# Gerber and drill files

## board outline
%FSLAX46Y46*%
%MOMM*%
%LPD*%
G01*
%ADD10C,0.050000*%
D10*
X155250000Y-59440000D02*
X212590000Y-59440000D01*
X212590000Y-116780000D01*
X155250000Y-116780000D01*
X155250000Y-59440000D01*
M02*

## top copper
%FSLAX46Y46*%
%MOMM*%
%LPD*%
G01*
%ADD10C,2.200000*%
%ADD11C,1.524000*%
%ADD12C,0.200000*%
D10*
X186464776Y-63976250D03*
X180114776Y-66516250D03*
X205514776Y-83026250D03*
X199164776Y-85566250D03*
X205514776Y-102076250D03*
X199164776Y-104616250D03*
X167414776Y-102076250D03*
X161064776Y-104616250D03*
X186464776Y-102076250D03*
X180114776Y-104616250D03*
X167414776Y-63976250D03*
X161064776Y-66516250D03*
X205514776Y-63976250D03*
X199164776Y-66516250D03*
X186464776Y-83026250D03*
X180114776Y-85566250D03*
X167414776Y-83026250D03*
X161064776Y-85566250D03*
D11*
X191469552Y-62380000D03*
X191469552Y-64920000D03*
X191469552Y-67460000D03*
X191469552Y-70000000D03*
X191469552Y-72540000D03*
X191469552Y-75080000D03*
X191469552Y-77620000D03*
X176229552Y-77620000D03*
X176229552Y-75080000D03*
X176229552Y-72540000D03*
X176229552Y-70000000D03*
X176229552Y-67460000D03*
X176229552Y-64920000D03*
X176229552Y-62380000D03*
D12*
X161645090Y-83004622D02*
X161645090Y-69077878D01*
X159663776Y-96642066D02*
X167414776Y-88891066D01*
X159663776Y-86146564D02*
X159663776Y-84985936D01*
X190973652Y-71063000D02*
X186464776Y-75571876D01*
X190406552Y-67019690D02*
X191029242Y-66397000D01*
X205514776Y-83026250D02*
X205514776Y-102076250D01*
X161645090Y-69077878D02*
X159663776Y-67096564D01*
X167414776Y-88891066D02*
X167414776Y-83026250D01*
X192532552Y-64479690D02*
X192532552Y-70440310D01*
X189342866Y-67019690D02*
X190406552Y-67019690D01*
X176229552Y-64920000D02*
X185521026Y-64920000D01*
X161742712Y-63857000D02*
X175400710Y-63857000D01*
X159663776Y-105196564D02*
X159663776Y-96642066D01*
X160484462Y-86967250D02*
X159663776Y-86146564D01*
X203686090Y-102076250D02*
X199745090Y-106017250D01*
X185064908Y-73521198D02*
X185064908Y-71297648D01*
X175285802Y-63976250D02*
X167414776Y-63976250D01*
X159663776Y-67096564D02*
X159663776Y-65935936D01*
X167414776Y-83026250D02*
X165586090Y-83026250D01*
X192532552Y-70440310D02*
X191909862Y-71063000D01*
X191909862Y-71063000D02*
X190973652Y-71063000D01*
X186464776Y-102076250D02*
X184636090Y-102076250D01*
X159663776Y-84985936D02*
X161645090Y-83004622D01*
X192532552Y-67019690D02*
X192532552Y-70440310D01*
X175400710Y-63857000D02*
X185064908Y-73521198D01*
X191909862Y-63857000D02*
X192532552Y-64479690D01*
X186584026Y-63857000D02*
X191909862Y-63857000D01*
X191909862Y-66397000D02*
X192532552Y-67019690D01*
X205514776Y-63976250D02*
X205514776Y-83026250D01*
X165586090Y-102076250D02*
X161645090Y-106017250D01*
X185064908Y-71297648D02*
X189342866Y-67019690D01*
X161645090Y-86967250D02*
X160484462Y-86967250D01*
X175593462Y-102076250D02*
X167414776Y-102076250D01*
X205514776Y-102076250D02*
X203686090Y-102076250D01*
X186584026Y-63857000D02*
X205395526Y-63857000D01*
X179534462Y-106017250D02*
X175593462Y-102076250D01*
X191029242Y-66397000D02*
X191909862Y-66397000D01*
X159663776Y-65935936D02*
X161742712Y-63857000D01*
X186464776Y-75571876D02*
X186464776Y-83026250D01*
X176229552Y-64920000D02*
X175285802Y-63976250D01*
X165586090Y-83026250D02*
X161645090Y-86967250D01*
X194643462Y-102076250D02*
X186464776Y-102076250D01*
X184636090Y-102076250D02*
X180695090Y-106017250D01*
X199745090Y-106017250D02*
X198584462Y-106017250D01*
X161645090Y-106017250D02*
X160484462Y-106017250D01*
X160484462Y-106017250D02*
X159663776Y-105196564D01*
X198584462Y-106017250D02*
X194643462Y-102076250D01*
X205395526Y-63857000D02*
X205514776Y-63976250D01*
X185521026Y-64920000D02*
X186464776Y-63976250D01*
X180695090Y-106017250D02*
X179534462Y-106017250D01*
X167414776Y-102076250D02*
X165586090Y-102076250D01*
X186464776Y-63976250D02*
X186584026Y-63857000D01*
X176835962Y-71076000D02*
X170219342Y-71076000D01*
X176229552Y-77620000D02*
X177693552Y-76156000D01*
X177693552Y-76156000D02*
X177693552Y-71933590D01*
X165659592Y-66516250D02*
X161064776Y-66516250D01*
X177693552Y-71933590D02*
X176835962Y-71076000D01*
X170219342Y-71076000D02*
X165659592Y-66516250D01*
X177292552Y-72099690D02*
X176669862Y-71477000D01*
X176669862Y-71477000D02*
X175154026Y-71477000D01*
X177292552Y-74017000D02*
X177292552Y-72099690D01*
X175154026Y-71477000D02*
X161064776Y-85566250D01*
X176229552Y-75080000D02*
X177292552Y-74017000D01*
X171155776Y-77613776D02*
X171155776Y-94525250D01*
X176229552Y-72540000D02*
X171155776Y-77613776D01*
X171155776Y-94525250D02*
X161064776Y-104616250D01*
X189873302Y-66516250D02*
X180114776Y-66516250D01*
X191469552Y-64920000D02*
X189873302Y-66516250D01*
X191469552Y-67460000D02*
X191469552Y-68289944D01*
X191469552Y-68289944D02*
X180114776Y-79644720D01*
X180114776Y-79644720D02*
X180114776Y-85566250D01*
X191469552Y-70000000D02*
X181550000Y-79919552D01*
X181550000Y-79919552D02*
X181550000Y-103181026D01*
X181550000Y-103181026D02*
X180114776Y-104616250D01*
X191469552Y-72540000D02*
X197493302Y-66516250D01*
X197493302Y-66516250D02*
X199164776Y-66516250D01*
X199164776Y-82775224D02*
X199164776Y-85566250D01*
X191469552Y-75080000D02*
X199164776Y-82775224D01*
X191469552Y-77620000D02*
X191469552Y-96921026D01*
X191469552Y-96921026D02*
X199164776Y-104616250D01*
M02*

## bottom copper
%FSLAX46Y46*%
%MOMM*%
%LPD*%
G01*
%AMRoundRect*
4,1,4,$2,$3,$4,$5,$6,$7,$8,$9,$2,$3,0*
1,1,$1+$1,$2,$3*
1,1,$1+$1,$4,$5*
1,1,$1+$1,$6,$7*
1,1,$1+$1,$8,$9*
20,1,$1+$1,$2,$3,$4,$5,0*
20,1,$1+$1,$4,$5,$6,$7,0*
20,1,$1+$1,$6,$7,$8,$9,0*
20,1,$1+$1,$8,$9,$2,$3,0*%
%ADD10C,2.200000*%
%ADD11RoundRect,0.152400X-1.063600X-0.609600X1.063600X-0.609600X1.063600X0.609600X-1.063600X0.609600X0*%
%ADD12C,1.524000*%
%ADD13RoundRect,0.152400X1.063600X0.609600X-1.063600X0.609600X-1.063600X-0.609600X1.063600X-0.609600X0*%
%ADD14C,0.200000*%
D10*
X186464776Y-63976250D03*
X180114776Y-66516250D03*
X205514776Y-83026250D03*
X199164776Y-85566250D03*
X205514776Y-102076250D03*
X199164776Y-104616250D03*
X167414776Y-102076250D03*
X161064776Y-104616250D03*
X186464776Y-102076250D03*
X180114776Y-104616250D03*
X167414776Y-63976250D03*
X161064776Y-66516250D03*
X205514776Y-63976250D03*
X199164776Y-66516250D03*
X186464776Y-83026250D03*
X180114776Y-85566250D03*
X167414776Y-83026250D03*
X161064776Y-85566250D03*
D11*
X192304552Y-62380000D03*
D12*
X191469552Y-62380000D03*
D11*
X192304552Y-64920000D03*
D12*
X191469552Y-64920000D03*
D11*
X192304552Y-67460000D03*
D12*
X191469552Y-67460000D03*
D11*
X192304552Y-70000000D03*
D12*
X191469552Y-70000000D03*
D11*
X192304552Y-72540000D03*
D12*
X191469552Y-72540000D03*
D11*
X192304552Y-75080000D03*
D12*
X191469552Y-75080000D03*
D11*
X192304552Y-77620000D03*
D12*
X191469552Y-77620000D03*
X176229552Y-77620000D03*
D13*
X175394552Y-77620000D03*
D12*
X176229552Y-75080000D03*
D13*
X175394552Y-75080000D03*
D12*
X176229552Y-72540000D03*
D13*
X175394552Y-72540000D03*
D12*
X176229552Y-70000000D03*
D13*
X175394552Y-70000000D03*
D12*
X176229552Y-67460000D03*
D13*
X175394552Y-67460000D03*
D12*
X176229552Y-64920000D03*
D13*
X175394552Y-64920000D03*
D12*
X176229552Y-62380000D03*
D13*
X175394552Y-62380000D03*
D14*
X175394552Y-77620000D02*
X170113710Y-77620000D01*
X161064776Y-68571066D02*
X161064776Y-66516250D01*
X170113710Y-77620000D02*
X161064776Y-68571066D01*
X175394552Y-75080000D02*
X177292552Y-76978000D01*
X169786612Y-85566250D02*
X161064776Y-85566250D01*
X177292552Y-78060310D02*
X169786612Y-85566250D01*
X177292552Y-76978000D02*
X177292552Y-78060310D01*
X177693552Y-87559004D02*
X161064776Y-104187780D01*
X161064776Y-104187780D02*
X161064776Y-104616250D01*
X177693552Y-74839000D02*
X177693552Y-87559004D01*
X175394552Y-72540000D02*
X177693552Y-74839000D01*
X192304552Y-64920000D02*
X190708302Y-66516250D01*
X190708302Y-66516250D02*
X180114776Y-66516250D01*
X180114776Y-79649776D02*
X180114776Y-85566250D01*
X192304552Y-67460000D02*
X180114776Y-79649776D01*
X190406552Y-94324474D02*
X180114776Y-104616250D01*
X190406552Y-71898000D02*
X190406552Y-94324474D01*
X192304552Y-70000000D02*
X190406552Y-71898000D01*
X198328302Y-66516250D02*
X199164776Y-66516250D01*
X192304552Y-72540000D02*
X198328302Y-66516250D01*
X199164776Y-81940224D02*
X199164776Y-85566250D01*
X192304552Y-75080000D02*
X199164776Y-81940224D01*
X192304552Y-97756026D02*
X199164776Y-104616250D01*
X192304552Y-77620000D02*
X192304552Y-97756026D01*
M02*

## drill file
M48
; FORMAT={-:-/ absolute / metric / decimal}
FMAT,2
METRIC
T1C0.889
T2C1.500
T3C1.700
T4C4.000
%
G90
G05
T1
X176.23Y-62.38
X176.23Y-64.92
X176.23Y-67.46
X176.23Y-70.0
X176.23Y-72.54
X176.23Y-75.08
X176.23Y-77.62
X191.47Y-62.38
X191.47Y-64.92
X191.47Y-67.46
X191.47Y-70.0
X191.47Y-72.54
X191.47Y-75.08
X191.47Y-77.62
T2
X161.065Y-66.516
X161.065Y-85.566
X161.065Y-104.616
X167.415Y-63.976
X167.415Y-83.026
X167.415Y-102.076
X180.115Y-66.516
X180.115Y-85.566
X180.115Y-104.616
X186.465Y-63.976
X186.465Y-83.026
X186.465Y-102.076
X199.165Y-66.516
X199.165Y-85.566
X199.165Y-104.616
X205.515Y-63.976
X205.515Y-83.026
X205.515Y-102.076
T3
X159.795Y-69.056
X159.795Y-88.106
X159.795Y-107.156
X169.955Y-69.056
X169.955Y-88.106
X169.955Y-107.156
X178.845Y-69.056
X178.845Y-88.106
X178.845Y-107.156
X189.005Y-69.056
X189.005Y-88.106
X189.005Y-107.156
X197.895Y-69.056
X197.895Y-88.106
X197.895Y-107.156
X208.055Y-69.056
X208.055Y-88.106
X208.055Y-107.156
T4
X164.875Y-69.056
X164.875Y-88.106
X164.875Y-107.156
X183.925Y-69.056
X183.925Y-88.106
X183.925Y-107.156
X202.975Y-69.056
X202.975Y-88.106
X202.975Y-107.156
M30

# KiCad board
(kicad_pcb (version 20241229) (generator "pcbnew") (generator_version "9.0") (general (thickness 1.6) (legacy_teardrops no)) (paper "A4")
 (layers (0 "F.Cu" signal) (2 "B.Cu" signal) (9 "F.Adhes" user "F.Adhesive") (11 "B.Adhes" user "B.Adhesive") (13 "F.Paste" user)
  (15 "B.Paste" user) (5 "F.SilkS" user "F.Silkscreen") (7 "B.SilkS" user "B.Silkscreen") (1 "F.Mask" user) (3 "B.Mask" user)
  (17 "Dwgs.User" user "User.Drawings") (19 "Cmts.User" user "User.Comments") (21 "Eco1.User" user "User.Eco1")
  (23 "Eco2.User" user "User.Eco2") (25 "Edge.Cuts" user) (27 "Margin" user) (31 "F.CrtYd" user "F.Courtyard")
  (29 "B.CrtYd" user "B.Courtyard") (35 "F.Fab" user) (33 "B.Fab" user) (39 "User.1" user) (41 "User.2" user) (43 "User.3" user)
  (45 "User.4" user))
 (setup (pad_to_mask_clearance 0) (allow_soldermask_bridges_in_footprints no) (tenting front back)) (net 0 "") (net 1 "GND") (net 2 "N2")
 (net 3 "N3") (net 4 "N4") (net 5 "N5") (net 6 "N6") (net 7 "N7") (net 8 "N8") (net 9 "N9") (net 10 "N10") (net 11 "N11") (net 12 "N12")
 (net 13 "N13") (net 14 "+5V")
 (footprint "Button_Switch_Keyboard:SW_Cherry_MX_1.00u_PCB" (layer "F.Cu") (at 186.464776 63.97625)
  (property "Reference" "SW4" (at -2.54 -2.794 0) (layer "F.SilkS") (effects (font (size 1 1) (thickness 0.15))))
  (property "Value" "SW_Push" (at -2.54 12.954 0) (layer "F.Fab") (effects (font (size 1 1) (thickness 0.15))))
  (pad "" np_thru_hole circle (at -7.62 5.08) (size 1.7 1.7) (drill 1.7) (layers "*.Cu" "*.Mask"))
  (pad "" np_thru_hole circle (at -2.54 5.08) (size 4 4) (drill 4) (layers "*.Cu" "*.Mask"))
  (pad "" np_thru_hole circle (at 2.54 5.08) (size 1.7 1.7) (drill 1.7) (layers "*.Cu" "*.Mask"))
  (pad "1" thru_hole circle (at 0 0) (size 2.2 2.2) (drill 1.5) (layers "*.Cu" "*.Mask") (remove_unused_layers no) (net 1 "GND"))
  (pad "2" thru_hole circle (at -6.35 2.54) (size 2.2 2.2) (drill 1.5) (layers "*.Cu" "*.Mask") (remove_unused_layers no) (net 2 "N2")))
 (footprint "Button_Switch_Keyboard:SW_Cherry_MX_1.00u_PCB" (layer "F.Cu") (at 205.514776 83.02625)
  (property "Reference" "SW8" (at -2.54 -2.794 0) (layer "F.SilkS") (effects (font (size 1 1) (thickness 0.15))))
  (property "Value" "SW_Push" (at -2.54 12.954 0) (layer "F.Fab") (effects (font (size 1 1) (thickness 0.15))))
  (pad "" np_thru_hole circle (at -7.62 5.08) (size 1.7 1.7) (drill 1.7) (layers "*.Cu" "*.Mask"))
  (pad "" np_thru_hole circle (at -2.54 5.08) (size 4 4) (drill 4) (layers "*.Cu" "*.Mask"))
  (pad "" np_thru_hole circle (at 2.54 5.08) (size 1.7 1.7) (drill 1.7) (layers "*.Cu" "*.Mask"))
  (pad "1" thru_hole circle (at 0 0) (size 2.2 2.2) (drill 1.5) (layers "*.Cu" "*.Mask") (remove_unused_layers no) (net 1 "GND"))
  (pad "2" thru_hole circle (at -6.35 2.54) (size 2.2 2.2) (drill 1.5) (layers "*.Cu" "*.Mask") (remove_unused_layers no) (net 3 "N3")))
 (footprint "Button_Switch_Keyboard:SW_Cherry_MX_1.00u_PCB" (layer "F.Cu") (at 205.514776 102.07625)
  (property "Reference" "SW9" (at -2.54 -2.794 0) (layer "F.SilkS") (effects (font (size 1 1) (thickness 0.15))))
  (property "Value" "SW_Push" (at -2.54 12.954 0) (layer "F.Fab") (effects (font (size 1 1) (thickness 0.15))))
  (pad "" np_thru_hole circle (at -7.62 5.08) (size 1.7 1.7) (drill 1.7) (layers "*.Cu" "*.Mask"))
  (pad "" np_thru_hole circle (at -2.54 5.08) (size 4 4) (drill 4) (layers "*.Cu" "*.Mask"))
  (pad "" np_thru_hole circle (at 2.54 5.08) (size 1.7 1.7) (drill 1.7) (layers "*.Cu" "*.Mask"))
  (pad "1" thru_hole circle (at 0 0) (size 2.2 2.2) (drill 1.5) (layers "*.Cu" "*.Mask") (remove_unused_layers no) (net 1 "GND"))
  (pad "2" thru_hole circle (at -6.35 2.54) (size 2.2 2.2) (drill 1.5) (layers "*.Cu" "*.Mask") (remove_unused_layers no) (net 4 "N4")))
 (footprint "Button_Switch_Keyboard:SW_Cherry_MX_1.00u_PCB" (layer "F.Cu") (at 167.414776 102.07625)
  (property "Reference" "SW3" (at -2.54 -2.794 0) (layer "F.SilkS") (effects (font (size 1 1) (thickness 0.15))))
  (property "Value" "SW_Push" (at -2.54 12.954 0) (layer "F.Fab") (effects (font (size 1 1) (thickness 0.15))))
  (pad "" np_thru_hole circle (at -7.62 5.08) (size 1.7 1.7) (drill 1.7) (layers "*.Cu" "*.Mask"))
  (pad "" np_thru_hole circle (at -2.54 5.08) (size 4 4) (drill 4) (layers "*.Cu" "*.Mask"))
  (pad "" np_thru_hole circle (at 2.54 5.08) (size 1.7 1.7) (drill 1.7) (layers "*.Cu" "*.Mask"))
  (pad "1" thru_hole circle (at 0 0) (size 2.2 2.2) (drill 1.5) (layers "*.Cu" "*.Mask") (remove_unused_layers no) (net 1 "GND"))
  (pad "2" thru_hole circle (at -6.35 2.54) (size 2.2 2.2) (drill 1.5) (layers "*.Cu" "*.Mask") (remove_unused_layers no) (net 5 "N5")))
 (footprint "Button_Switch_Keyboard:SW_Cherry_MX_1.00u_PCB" (layer "F.Cu") (at 186.464776 102.07625)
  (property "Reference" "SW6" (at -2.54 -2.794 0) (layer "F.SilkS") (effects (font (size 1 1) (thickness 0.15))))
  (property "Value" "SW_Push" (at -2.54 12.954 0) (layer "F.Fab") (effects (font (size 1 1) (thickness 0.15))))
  (pad "" np_thru_hole circle (at -7.62 5.08) (size 1.7 1.7) (drill 1.7) (layers "*.Cu" "*.Mask"))
  (pad "" np_thru_hole circle (at -2.54 5.08) (size 4 4) (drill 4) (layers "*.Cu" "*.Mask"))
  (pad "" np_thru_hole circle (at 2.54 5.08) (size 1.7 1.7) (drill 1.7) (layers "*.Cu" "*.Mask"))
  (pad "1" thru_hole circle (at 0 0) (size 2.2 2.2) (drill 1.5) (layers "*.Cu" "*.Mask") (remove_unused_layers no) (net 1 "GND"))
  (pad "2" thru_hole circle (at -6.35 2.54) (size 2.2 2.2) (drill 1.5) (layers "*.Cu" "*.Mask") (remove_unused_layers no) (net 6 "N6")))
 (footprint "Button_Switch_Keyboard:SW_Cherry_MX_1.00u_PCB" (layer "F.Cu") (at 167.414776 63.97625)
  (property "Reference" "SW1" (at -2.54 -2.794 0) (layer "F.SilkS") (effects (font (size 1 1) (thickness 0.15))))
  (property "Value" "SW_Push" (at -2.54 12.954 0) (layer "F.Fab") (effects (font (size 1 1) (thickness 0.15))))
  (pad "" np_thru_hole circle (at -7.62 5.08) (size 1.7 1.7) (drill 1.7) (layers "*.Cu" "*.Mask"))
  (pad "" np_thru_hole circle (at -2.54 5.08) (size 4 4) (drill 4) (layers "*.Cu" "*.Mask"))
  (pad "" np_thru_hole circle (at 2.54 5.08) (size 1.7 1.7) (drill 1.7) (layers "*.Cu" "*.Mask"))
  (pad "1" thru_hole circle (at 0 0) (size 2.2 2.2) (drill 1.5) (layers "*.Cu" "*.Mask") (remove_unused_layers no) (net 1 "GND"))
  (pad "2" thru_hole circle (at -6.35 2.54) (size 2.2 2.2) (drill 1.5) (layers "*.Cu" "*.Mask") (remove_unused_layers no) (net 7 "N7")))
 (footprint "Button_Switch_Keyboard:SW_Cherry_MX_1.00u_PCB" (layer "F.Cu") (at 205.514776 63.97625)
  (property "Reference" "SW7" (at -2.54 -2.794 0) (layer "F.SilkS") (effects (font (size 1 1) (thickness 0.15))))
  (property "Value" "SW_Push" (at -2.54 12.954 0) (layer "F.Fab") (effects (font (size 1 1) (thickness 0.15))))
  (pad "" np_thru_hole circle (at -7.62 5.08) (size 1.7 1.7) (drill 1.7) (layers "*.Cu" "*.Mask"))
  (pad "" np_thru_hole circle (at -2.54 5.08) (size 4 4) (drill 4) (layers "*.Cu" "*.Mask"))
  (pad "" np_thru_hole circle (at 2.54 5.08) (size 1.7 1.7) (drill 1.7) (layers "*.Cu" "*.Mask"))
  (pad "1" thru_hole circle (at 0 0) (size 2.2 2.2) (drill 1.5) (layers "*.Cu" "*.Mask") (remove_unused_layers no) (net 1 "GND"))
  (pad "2" thru_hole circle (at -6.35 2.54) (size 2.2 2.2) (drill 1.5) (layers "*.Cu" "*.Mask") (remove_unused_layers no) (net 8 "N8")))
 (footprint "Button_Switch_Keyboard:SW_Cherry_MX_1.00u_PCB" (layer "F.Cu") (at 186.464776 83.02625)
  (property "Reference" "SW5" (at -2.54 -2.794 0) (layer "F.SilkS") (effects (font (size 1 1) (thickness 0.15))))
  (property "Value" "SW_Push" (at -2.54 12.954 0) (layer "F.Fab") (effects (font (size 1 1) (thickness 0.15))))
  (pad "" np_thru_hole circle (at -7.62 5.08) (size 1.7 1.7) (drill 1.7) (layers "*.Cu" "*.Mask"))
  (pad "" np_thru_hole circle (at -2.54 5.08) (size 4 4) (drill 4) (layers "*.Cu" "*.Mask"))
  (pad "" np_thru_hole circle (at 2.54 5.08) (size 1.7 1.7) (drill 1.7) (layers "*.Cu" "*.Mask"))
  (pad "1" thru_hole circle (at 0 0) (size 2.2 2.2) (drill 1.5) (layers "*.Cu" "*.Mask") (remove_unused_layers no) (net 1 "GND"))
  (pad "2" thru_hole circle (at -6.35 2.54) (size 2.2 2.2) (drill 1.5) (layers "*.Cu" "*.Mask") (remove_unused_layers no) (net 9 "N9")))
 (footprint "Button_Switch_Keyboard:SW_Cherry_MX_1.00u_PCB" (layer "F.Cu") (at 167.414776 83.02625)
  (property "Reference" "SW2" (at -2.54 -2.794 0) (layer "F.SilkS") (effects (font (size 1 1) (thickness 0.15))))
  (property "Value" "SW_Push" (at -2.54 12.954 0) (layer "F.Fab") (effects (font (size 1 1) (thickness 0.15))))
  (pad "" np_thru_hole circle (at -7.62 5.08) (size 1.7 1.7) (drill 1.7) (layers "*.Cu" "*.Mask"))
  (pad "" np_thru_hole circle (at -2.54 5.08) (size 4 4) (drill 4) (layers "*.Cu" "*.Mask"))
  (pad "" np_thru_hole circle (at 2.54 5.08) (size 1.7 1.7) (drill 1.7) (layers "*.Cu" "*.Mask"))
  (pad "1" thru_hole circle (at 0 0) (size 2.2 2.2) (drill 1.5) (layers "*.Cu" "*.Mask") (remove_unused_layers no) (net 1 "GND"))
  (pad "2" thru_hole circle (at -6.35 2.54) (size 2.2 2.2) (drill 1.5) (layers "*.Cu" "*.Mask") (remove_unused_layers no) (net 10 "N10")))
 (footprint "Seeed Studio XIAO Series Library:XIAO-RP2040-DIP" (layer "B.Cu") (at 183.849552 70 180)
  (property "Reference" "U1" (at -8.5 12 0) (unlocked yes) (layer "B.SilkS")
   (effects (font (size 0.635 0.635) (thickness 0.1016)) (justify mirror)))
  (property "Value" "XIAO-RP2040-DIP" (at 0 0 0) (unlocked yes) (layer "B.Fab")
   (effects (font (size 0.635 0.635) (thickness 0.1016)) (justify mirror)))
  (pad "1" smd roundrect (at -8.455 7.62) (size 2.432 1.524) (layers "B.Cu" "B.Mask") (roundrect_rratio 0.1) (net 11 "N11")
   (thermal_bridge_angle 45))
  (pad "1" thru_hole circle (at -7.62 7.62) (size 1.524 1.524) (drill 0.889) (layers "*.Cu" "*.Mask") (remove_unused_layers no)
   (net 11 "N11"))
  (pad "2" smd roundrect (at -8.455 5.08) (size 2.432 1.524) (layers "B.Cu" "B.Mask") (roundrect_rratio 0.1) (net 2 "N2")
   (thermal_bridge_angle 45))
  (pad "2" thru_hole circle (at -7.62 5.08) (size 1.524 1.524) (drill 0.889) (layers "*.Cu" "*.Mask") (remove_unused_layers no) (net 2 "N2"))
  (pad "3" smd roundrect (at -8.455 2.54) (size 2.432 1.524) (layers "B.Cu" "B.Mask") (roundrect_rratio 0.1) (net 9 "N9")
   (thermal_bridge_angle 45))
  (pad "3" thru_hole circle (at -7.62 2.54) (size 1.524 1.524) (drill 0.889) (layers "*.Cu" "*.Mask") (remove_unused_layers no) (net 9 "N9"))
  (pad "4" smd roundrect (at -8.455 0) (size 2.432 1.524) (layers "B.Cu" "B.Mask") (roundrect_rratio 0.1) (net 6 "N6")
   (thermal_bridge_angle 45))
  (pad "4" thru_hole circle (at -7.62 0) (size 1.524 1.524) (drill 0.889) (layers "*.Cu" "*.Mask") (remove_unused_layers no) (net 6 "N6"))
  (pad "5" smd roundrect (at -8.455 -2.54) (size 2.432 1.524) (layers "B.Cu" "B.Mask") (roundrect_rratio 0.1) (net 8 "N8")
   (thermal_bridge_angle 45))
  (pad "5" thru_hole circle (at -7.62 -2.54) (size 1.524 1.524) (drill 0.889) (layers "*.Cu" "*.Mask") (remove_unused_layers no)
   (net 8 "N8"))
  (pad "6" smd roundrect (at -8.455 -5.08) (size 2.432 1.524) (layers "B.Cu" "B.Mask") (roundrect_rratio 0.1) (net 3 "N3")
   (thermal_bridge_angle 45))
  (pad "6" thru_hole circle (at -7.62 -5.08) (size 1.524 1.524) (drill 0.889) (layers "*.Cu" "*.Mask") (remove_unused_layers no)
   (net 3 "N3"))
  (pad "7" smd roundrect (at -8.455 -7.62) (size 2.432 1.524) (layers "B.Cu" "B.Mask") (roundrect_rratio 0.1) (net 4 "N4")
   (thermal_bridge_angle 45))
  (pad "7" thru_hole circle (at -7.62 -7.62) (size 1.524 1.524) (drill 0.889) (layers "*.Cu" "*.Mask") (remove_unused_layers no)
   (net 4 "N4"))
  (pad "8" thru_hole circle (at 7.62 -7.62 180) (size 1.524 1.524) (drill 0.889) (layers "*.Cu" "*.Mask") (remove_unused_layers no)
   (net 7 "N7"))
  (pad "8" smd roundrect (at 8.455 -7.62 180) (size 2.432 1.524) (layers "B.Cu" "B.Mask") (roundrect_rratio 0.1) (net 7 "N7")
   (thermal_bridge_angle 45))
  (pad "9" thru_hole circle (at 7.62 -5.08 180) (size 1.524 1.524) (drill 0.889) (layers "*.Cu" "*.Mask") (remove_unused_layers no)
   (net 10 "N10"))
  (pad "9" smd roundrect (at 8.455 -5.08 180) (size 2.432 1.524) (layers "B.Cu" "B.Mask") (roundrect_rratio 0.1) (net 10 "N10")
   (thermal_bridge_angle 45))
  (pad "10" thru_hole circle (at 7.62 -2.54 180) (size 1.524 1.524) (drill 0.889) (layers "*.Cu" "*.Mask") (remove_unused_layers no)
   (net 5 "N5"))
  (pad "10" smd roundrect (at 8.455 -2.54 180) (size 2.432 1.524) (layers "B.Cu" "B.Mask") (roundrect_rratio 0.1) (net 5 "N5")
   (thermal_bridge_angle 45))
  (pad "11" thru_hole circle (at 7.62 0 180) (size 1.524 1.524) (drill 0.889) (layers "*.Cu" "*.Mask") (remove_unused_layers no)
   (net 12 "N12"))
  (pad "11" smd roundrect (at 8.455 0 180) (size 2.432 1.524) (layers "B.Cu" "B.Mask") (roundrect_rratio 0.1) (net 12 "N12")
   (thermal_bridge_angle 45))
  (pad "12" thru_hole circle (at 7.62 2.54 180) (size 1.524 1.524) (drill 0.889) (layers "*.Cu" "*.Mask") (remove_unused_layers no)
   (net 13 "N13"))
  (pad "12" smd roundrect (at 8.455 2.54 180) (size 2.432 1.524) (layers "B.Cu" "B.Mask") (roundrect_rratio 0.1) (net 13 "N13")
   (thermal_bridge_angle 45))
  (pad "13" thru_hole circle (at 7.62 5.08 180) (size 1.524 1.524) (drill 0.889) (layers "*.Cu" "*.Mask") (remove_unused_layers no)
   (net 1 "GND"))
  (pad "13" smd roundrect (at 8.455 5.08 180) (size 2.432 1.524) (layers "B.Cu" "B.Mask") (roundrect_rratio 0.1) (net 1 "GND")
   (thermal_bridge_angle 45))
  (pad "14" thru_hole circle (at 7.62 7.62 180) (size 1.524 1.524) (drill 0.889) (layers "*.Cu" "*.Mask") (remove_unused_layers no)
   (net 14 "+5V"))
  (pad "14" smd roundrect (at 8.455 7.62 180) (size 2.432 1.524) (layers "B.Cu" "B.Mask") (roundrect_rratio 0.1) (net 14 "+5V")
   (thermal_bridge_angle 45)))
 (gr_rect (start 155.25 59.44) (end 212.59 116.78) (stroke (width 0.05) (type default)) (fill no) (layer "Edge.Cuts"))
 (segment (start 161.64509 83.004622) (end 161.64509 69.077878) (width 0.2) (layer "F.Cu") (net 1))
 (segment (start 159.663776 96.642066) (end 167.414776 88.891066) (width 0.2) (layer "F.Cu") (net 1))
 (segment (start 159.663776 86.146564) (end 159.663776 84.985936) (width 0.2) (layer "F.Cu") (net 1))
 (segment (start 190.973652 71.063) (end 186.464776 75.571876) (width 0.2) (layer "F.Cu") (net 1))
 (segment (start 190.406552 67.01969) (end 191.029242 66.397) (width 0.2) (layer "F.Cu") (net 1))
 (segment (start 205.514776 83.02625) (end 205.514776 102.07625) (width 0.2) (layer "F.Cu") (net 1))
 (segment (start 161.64509 69.077878) (end 159.663776 67.096564) (width 0.2) (layer "F.Cu") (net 1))
 (segment (start 167.414776 88.891066) (end 167.414776 83.02625) (width 0.2) (layer "F.Cu") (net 1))
 (segment (start 192.532552 64.47969) (end 192.532552 70.44031) (width 0.2) (layer "F.Cu") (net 1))
 (segment (start 189.342866 67.01969) (end 190.406552 67.01969) (width 0.2) (layer "F.Cu") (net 1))
 (segment (start 176.229552 64.92) (end 185.521026 64.92) (width 0.2) (layer "F.Cu") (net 1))
 (segment (start 161.742712 63.857) (end 175.40071 63.857) (width 0.2) (layer "F.Cu") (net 1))
 (segment (start 159.663776 105.196564) (end 159.663776 96.642066) (width 0.2) (layer "F.Cu") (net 1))
 (segment (start 160.484462 86.96725) (end 159.663776 86.146564) (width 0.2) (layer "F.Cu") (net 1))
 (segment (start 203.68609 102.07625) (end 199.74509 106.01725) (width 0.2) (layer "F.Cu") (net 1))
 (segment (start 185.064908 73.521198) (end 185.064908 71.297648) (width 0.2) (layer "F.Cu") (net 1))
 (segment (start 175.285802 63.97625) (end 167.414776 63.97625) (width 0.2) (layer "F.Cu") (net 1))
 (segment (start 159.663776 67.096564) (end 159.663776 65.935936) (width 0.2) (layer "F.Cu") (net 1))
 (segment (start 167.414776 83.02625) (end 165.58609 83.02625) (width 0.2) (layer "F.Cu") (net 1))
 (segment (start 192.532552 70.44031) (end 191.909862 71.063) (width 0.2) (layer "F.Cu") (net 1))
 (segment (start 191.909862 71.063) (end 190.973652 71.063) (width 0.2) (layer "F.Cu") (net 1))
 (segment (start 186.464776 102.07625) (end 184.63609 102.07625) (width 0.2) (layer "F.Cu") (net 1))
 (segment (start 159.663776 84.985936) (end 161.64509 83.004622) (width 0.2) (layer "F.Cu") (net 1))
 (segment (start 192.532552 67.01969) (end 192.532552 70.44031) (width 0.2) (layer "F.Cu") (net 1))
 (segment (start 175.40071 63.857) (end 185.064908 73.521198) (width 0.2) (layer "F.Cu") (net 1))
 (segment (start 191.909862 63.857) (end 192.532552 64.47969) (width 0.2) (layer "F.Cu") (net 1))
 (segment (start 186.584026 63.857) (end 191.909862 63.857) (width 0.2) (layer "F.Cu") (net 1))
 (segment (start 191.909862 66.397) (end 192.532552 67.01969) (width 0.2) (layer "F.Cu") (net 1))
 (segment (start 205.514776 63.97625) (end 205.514776 83.02625) (width 0.2) (layer "F.Cu") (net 1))
 (segment (start 165.58609 102.07625) (end 161.64509 106.01725) (width 0.2) (layer "F.Cu") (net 1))
 (segment (start 185.064908 71.297648) (end 189.342866 67.01969) (width 0.2) (layer "F.Cu") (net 1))
 (segment (start 161.64509 86.96725) (end 160.484462 86.96725) (width 0.2) (layer "F.Cu") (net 1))
 (segment (start 175.593462 102.07625) (end 167.414776 102.07625) (width 0.2) (layer "F.Cu") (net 1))
 (segment (start 205.514776 102.07625) (end 203.68609 102.07625) (width 0.2) (layer "F.Cu") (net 1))
 (segment (start 186.584026 63.857) (end 205.395526 63.857) (width 0.2) (layer "F.Cu") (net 1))
 (segment (start 179.534462 106.01725) (end 175.593462 102.07625) (width 0.2) (layer "F.Cu") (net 1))
 (segment (start 191.029242 66.397) (end 191.909862 66.397) (width 0.2) (layer "F.Cu") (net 1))
 (segment (start 159.663776 65.935936) (end 161.742712 63.857) (width 0.2) (layer "F.Cu") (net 1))
 (segment (start 186.464776 75.571876) (end 186.464776 83.02625) (width 0.2) (layer "F.Cu") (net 1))
 (segment (start 176.229552 64.92) (end 175.285802 63.97625) (width 0.2) (layer "F.Cu") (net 1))
 (segment (start 165.58609 83.02625) (end 161.64509 86.96725) (width 0.2) (layer "F.Cu") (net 1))
 (segment (start 194.643462 102.07625) (end 186.464776 102.07625) (width 0.2) (layer "F.Cu") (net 1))
 (segment (start 184.63609 102.07625) (end 180.69509 106.01725) (width 0.2) (layer "F.Cu") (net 1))
 (segment (start 199.74509 106.01725) (end 198.584462 106.01725) (width 0.2) (layer "F.Cu") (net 1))
 (segment (start 161.64509 106.01725) (end 160.484462 106.01725) (width 0.2) (layer "F.Cu") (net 1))
 (segment (start 160.484462 106.01725) (end 159.663776 105.196564) (width 0.2) (layer "F.Cu") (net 1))
 (segment (start 198.584462 106.01725) (end 194.643462 102.07625) (width 0.2) (layer "F.Cu") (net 1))
 (segment (start 205.395526 63.857) (end 205.514776 63.97625) (width 0.2) (layer "F.Cu") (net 1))
 (segment (start 185.521026 64.92) (end 186.464776 63.97625) (width 0.2) (layer "F.Cu") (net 1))
 (segment (start 180.69509 106.01725) (end 179.534462 106.01725) (width 0.2) (layer "F.Cu") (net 1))
 (segment (start 167.414776 102.07625) (end 165.58609 102.07625) (width 0.2) (layer "F.Cu") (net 1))
 (segment (start 186.464776 63.97625) (end 186.584026 63.857) (width 0.2) (layer "F.Cu") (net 1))
 (segment (start 176.835962 71.076) (end 170.219342 71.076) (width 0.2) (layer "F.Cu") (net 7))
 (segment (start 176.229552 77.62) (end 177.693552 76.156) (width 0.2) (layer "F.Cu") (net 7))
 (segment (start 177.693552 76.156) (end 177.693552 71.93359) (width 0.2) (layer "F.Cu") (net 7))
 (segment (start 165.659592 66.51625) (end 161.064776 66.51625) (width 0.2) (layer "F.Cu") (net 7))
 (segment (start 177.693552 71.93359) (end 176.835962 71.076) (width 0.2) (layer "F.Cu") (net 7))
 (segment (start 170.219342 71.076) (end 165.659592 66.51625) (width 0.2) (layer "F.Cu") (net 7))
 (segment (start 175.394552 77.62) (end 170.11371 77.62) (width 0.2) (layer "B.Cu") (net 7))
 (segment (start 161.064776 68.571066) (end 161.064776 66.51625) (width 0.2) (layer "B.Cu") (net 7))
 (segment (start 170.11371 77.62) (end 161.064776 68.571066) (width 0.2) (layer "B.Cu") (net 7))
 (segment (start 177.292552 72.09969) (end 176.669862 71.477) (width 0.2) (layer "F.Cu") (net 10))
 (segment (start 176.669862 71.477) (end 175.154026 71.477) (width 0.2) (layer "F.Cu") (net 10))
 (segment (start 177.292552 74.017) (end 177.292552 72.09969) (width 0.2) (layer "F.Cu") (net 10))
 (segment (start 175.154026 71.477) (end 161.064776 85.56625) (width 0.2) (layer "F.Cu") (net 10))
 (segment (start 176.229552 75.08) (end 177.292552 74.017) (width 0.2) (layer "F.Cu") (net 10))
 (segment (start 175.394552 75.08) (end 177.292552 76.978) (width 0.2) (layer "B.Cu") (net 10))
 (segment (start 169.786612 85.56625) (end 161.064776 85.56625) (width 0.2) (layer "B.Cu") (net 10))
 (segment (start 177.292552 78.06031) (end 169.786612 85.56625) (width 0.2) (layer "B.Cu") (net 10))
 (segment (start 177.292552 76.978) (end 177.292552 78.06031) (width 0.2) (layer "B.Cu") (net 10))
 (segment (start 171.155776 77.613776) (end 171.155776 94.52525) (width 0.2) (layer "F.Cu") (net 5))
 (segment (start 176.229552 72.54) (end 171.155776 77.613776) (width 0.2) (layer "F.Cu") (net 5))
 (segment (start 171.155776 94.52525) (end 161.064776 104.61625) (width 0.2) (layer "F.Cu") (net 5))
 (segment (start 177.693552 87.559004) (end 161.064776 104.18778) (width 0.2) (layer "B.Cu") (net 5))
 (segment (start 161.064776 104.18778) (end 161.064776 104.61625) (width 0.2) (layer "B.Cu") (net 5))
 (segment (start 177.693552 74.839) (end 177.693552 87.559004) (width 0.2) (layer "B.Cu") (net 5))
 (segment (start 175.394552 72.54) (end 177.693552 74.839) (width 0.2) (layer "B.Cu") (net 5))
 (segment (start 189.873302 66.51625) (end 180.114776 66.51625) (width 0.2) (layer "F.Cu") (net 2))
 (segment (start 191.469552 64.92) (end 189.873302 66.51625) (width 0.2) (layer "F.Cu") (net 2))
 (segment (start 192.304552 64.92) (end 190.708302 66.51625) (width 0.2) (layer "B.Cu") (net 2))
 (segment (start 190.708302 66.51625) (end 180.114776 66.51625) (width 0.2) (layer "B.Cu") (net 2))
 (segment (start 191.469552 67.46) (end 191.469552 68.289944) (width 0.2) (layer "F.Cu") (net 9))
 (segment (start 191.469552 68.289944) (end 180.114776 79.64472) (width 0.2) (layer "F.Cu") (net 9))
 (segment (start 180.114776 79.64472) (end 180.114776 85.56625) (width 0.2) (layer "F.Cu") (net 9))
 (segment (start 180.114776 79.649776) (end 180.114776 85.56625) (width 0.2) (layer "B.Cu") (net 9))
 (segment (start 192.304552 67.46) (end 180.114776 79.649776) (width 0.2) (layer "B.Cu") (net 9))
 (segment (start 191.469552 70) (end 181.55 79.919552) (width 0.2) (layer "F.Cu") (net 6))
 (segment (start 181.55 79.919552) (end 181.55 103.181026) (width 0.2) (layer "F.Cu") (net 6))
 (segment (start 181.55 103.181026) (end 180.114776 104.61625) (width 0.2) (layer "F.Cu") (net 6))
 (segment (start 190.406552 94.324474) (end 180.114776 104.61625) (width 0.2) (layer "B.Cu") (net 6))
 (segment (start 190.406552 71.898) (end 190.406552 94.324474) (width 0.2) (layer "B.Cu") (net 6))
 (segment (start 192.304552 70) (end 190.406552 71.898) (width 0.2) (layer "B.Cu") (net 6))
 (segment (start 191.469552 72.54) (end 197.493302 66.51625) (width 0.2) (layer "F.Cu") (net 8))
 (segment (start 197.493302 66.51625) (end 199.164776 66.51625) (width 0.2) (layer "F.Cu") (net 8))
 (segment (start 198.328302 66.51625) (end 199.164776 66.51625) (width 0.2) (layer "B.Cu") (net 8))
 (segment (start 192.304552 72.54) (end 198.328302 66.51625) (width 0.2) (layer "B.Cu") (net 8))
 (segment (start 199.164776 82.775224) (end 199.164776 85.56625) (width 0.2) (layer "F.Cu") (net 3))
 (segment (start 191.469552 75.08) (end 199.164776 82.775224) (width 0.2) (layer "F.Cu") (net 3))
 (segment (start 199.164776 81.940224) (end 199.164776 85.56625) (width 0.2) (layer "B.Cu") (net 3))
 (segment (start 192.304552 75.08) (end 199.164776 81.940224) (width 0.2) (layer "B.Cu") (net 3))
 (segment (start 191.469552 77.62) (end 191.469552 96.921026) (width 0.2) (layer "F.Cu") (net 4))
 (segment (start 191.469552 96.921026) (end 199.164776 104.61625) (width 0.2) (layer "F.Cu") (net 4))
 (segment (start 192.304552 97.756026) (end 199.164776 104.61625) (width 0.2) (layer "B.Cu") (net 4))
 (segment (start 192.304552 77.62) (end 192.304552 97.756026) (width 0.2) (layer "B.Cu") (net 4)))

